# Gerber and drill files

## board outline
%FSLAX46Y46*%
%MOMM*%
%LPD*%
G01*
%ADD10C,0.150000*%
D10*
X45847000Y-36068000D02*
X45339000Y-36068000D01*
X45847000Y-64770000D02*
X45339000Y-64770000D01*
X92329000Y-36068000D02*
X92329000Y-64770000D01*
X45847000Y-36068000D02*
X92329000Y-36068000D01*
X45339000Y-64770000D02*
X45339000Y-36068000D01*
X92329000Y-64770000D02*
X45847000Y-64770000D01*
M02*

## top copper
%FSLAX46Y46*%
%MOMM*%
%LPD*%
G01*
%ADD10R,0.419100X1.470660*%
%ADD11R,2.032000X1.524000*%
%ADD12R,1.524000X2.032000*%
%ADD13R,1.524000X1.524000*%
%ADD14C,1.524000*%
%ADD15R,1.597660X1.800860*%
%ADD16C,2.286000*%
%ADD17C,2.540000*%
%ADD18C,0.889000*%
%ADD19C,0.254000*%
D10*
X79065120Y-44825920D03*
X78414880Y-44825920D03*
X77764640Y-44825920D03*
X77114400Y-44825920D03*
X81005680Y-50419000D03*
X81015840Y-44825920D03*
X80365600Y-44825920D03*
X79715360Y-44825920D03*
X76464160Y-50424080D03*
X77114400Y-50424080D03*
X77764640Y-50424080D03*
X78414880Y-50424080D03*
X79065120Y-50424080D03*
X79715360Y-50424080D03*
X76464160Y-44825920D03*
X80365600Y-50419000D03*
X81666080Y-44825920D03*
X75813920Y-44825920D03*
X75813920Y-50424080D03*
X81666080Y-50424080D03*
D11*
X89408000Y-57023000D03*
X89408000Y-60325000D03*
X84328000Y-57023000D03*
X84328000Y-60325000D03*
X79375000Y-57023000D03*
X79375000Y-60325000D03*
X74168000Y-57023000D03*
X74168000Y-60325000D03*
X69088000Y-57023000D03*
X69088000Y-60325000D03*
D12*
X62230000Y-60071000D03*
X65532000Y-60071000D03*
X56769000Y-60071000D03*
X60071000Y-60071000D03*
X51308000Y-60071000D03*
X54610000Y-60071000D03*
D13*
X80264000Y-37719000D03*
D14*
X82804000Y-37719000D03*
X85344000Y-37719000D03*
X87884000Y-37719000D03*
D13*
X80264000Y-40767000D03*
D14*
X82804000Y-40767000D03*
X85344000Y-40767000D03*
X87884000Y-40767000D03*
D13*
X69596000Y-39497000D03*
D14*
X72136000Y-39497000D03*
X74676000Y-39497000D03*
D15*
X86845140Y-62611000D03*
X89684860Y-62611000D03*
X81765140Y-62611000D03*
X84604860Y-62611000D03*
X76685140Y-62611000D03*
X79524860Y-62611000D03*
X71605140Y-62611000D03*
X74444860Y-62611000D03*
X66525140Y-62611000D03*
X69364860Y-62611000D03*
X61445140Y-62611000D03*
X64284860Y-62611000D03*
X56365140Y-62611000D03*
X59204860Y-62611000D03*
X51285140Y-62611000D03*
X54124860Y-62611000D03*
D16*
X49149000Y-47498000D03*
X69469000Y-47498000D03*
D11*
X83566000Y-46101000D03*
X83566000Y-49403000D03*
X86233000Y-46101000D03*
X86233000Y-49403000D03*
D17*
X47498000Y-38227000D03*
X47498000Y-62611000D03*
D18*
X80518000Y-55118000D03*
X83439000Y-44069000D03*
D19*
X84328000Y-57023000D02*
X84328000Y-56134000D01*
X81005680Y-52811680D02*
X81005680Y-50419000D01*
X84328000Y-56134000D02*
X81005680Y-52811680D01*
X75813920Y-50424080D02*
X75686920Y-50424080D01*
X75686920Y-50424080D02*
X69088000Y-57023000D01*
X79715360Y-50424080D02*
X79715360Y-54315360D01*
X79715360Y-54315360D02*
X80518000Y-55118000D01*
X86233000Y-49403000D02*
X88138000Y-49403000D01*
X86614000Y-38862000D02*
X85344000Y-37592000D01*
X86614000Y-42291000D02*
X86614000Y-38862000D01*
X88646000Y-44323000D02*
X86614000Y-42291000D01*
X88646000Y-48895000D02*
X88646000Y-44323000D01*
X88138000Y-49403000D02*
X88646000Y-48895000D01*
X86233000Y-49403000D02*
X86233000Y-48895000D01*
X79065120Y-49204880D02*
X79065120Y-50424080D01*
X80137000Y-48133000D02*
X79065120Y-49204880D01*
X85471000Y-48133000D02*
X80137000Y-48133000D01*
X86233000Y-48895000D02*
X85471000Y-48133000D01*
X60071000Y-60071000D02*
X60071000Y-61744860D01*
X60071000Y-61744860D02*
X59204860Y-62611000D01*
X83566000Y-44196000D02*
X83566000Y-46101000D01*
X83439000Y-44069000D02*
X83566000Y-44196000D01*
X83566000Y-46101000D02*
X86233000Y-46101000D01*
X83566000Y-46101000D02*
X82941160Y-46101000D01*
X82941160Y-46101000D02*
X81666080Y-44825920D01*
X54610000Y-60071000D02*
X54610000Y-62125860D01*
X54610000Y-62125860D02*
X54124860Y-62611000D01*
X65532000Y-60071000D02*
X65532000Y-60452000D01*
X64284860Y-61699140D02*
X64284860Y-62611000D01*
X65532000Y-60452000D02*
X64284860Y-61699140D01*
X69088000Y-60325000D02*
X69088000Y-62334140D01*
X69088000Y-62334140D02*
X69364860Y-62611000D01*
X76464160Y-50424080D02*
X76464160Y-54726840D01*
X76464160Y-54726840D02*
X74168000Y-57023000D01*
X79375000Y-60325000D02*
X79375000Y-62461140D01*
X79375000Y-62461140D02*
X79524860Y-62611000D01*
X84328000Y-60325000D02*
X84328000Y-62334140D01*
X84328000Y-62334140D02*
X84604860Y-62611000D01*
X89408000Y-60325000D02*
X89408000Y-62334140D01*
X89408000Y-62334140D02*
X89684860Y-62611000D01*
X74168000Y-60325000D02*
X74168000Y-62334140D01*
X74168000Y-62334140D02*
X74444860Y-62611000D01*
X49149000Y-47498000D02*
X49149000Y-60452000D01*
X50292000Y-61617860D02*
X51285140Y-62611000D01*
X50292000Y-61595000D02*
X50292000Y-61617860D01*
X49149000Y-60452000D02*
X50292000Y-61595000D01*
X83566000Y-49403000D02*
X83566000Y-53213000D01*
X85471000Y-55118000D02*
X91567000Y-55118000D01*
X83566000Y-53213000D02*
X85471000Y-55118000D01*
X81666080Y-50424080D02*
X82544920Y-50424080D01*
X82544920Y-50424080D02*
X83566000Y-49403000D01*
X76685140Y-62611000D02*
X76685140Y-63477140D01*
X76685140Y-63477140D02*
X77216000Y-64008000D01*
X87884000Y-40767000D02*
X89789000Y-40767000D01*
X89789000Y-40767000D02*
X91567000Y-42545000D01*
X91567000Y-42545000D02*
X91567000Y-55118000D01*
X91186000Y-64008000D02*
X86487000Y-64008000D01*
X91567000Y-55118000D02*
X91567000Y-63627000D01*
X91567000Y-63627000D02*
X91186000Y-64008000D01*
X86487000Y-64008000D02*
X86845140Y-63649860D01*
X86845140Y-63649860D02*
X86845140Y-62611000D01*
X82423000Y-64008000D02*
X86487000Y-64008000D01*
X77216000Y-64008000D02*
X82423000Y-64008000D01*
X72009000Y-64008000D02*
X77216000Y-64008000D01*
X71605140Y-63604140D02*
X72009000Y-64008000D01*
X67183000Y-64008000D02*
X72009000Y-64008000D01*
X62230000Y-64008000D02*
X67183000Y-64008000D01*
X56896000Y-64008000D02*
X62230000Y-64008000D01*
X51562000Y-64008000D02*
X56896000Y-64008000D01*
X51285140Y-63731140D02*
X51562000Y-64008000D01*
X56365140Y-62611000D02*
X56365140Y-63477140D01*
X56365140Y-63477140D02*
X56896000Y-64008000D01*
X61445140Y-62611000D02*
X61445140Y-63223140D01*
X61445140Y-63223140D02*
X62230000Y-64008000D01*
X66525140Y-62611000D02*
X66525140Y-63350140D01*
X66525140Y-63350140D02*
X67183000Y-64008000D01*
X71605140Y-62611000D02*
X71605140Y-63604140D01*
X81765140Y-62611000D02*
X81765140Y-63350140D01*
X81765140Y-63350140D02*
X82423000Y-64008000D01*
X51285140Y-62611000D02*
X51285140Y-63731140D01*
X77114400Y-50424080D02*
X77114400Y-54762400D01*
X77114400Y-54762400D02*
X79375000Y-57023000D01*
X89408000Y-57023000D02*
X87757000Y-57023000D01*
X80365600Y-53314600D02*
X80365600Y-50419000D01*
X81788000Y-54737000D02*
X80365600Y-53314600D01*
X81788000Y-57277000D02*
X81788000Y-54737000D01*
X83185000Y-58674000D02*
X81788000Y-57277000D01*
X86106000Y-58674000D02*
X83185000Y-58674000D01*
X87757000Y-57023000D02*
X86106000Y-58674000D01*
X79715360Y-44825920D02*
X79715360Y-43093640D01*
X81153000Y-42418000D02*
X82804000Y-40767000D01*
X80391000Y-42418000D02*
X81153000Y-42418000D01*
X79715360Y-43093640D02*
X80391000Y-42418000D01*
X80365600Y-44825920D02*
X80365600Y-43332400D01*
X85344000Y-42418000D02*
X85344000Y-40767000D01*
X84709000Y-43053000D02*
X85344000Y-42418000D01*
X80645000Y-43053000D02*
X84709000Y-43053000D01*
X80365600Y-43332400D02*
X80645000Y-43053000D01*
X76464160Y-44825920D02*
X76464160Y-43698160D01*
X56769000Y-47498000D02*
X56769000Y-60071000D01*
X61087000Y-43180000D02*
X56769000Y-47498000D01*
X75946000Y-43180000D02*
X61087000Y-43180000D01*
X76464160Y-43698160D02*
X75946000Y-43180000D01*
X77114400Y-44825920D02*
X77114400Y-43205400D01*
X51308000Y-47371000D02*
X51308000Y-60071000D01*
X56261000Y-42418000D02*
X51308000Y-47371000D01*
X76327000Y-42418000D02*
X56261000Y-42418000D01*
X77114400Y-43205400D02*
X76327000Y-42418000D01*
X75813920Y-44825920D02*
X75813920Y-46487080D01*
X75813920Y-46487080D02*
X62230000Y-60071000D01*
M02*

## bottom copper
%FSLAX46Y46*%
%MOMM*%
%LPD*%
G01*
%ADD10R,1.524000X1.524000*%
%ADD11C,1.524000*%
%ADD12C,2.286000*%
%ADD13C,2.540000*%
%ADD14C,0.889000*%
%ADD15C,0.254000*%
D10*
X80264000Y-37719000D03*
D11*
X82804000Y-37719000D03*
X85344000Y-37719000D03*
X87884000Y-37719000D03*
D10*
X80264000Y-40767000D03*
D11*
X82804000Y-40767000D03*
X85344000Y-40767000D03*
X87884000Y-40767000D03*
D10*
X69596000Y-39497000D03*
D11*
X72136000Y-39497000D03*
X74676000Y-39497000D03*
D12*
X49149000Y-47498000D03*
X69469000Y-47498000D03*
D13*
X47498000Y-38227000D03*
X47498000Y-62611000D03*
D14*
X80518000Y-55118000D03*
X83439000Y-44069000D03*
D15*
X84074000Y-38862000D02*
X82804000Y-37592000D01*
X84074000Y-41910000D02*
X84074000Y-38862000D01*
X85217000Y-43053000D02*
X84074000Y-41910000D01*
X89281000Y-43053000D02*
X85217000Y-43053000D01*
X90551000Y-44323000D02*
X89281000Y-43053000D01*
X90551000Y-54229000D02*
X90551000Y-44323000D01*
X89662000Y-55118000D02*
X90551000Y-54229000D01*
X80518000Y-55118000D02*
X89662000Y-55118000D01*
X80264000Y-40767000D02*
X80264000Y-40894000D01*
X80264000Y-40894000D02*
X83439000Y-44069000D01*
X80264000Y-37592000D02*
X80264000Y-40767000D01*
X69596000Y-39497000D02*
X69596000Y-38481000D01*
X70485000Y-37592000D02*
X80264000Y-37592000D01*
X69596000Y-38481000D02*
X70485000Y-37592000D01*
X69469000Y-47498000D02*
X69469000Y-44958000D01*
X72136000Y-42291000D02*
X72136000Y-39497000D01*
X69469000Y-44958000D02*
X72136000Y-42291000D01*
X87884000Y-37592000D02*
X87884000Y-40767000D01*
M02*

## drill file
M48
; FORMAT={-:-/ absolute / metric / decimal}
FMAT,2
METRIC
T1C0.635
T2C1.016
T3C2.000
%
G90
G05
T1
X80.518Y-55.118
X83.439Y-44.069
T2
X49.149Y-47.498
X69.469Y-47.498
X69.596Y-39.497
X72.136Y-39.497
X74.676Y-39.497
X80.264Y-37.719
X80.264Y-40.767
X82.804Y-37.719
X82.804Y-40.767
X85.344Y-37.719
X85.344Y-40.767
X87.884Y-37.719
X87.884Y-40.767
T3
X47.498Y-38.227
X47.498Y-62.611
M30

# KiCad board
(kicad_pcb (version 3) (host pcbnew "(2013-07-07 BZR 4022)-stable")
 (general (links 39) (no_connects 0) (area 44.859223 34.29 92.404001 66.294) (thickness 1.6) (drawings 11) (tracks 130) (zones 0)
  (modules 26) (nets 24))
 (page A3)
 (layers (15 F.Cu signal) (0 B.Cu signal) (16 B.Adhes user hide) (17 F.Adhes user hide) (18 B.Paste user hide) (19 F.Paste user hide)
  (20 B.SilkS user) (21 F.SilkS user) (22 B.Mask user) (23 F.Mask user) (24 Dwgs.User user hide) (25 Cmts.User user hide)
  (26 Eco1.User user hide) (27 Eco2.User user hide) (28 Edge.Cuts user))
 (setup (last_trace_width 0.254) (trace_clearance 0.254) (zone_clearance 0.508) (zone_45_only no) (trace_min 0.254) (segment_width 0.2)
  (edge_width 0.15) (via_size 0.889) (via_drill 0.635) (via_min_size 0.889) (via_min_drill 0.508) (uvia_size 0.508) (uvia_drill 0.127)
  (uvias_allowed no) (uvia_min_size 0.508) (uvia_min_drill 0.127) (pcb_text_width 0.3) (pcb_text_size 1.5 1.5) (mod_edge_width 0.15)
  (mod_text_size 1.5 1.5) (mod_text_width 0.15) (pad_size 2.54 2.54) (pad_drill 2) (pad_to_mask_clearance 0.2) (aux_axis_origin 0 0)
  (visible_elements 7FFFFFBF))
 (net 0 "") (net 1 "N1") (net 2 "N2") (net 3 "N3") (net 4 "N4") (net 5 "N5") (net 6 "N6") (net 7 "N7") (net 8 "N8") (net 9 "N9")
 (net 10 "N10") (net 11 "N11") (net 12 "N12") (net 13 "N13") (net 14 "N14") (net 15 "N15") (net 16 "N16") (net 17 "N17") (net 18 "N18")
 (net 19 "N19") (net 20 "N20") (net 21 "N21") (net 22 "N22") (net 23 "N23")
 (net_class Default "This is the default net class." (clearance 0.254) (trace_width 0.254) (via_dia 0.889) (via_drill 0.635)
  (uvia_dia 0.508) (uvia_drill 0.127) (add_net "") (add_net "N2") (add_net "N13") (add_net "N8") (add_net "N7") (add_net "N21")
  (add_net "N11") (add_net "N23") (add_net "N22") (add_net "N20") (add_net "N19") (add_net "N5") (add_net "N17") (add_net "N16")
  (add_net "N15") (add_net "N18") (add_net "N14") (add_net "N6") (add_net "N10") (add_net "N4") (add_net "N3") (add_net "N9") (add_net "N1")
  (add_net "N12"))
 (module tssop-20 (layer F.Cu) (at 78.74 47.625 180)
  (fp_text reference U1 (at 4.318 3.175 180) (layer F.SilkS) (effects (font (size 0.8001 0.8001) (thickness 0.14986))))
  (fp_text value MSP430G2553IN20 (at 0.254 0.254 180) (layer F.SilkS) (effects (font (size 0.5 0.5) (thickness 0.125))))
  (pad 5 smd rect (at -0.32512 2.79908 180) (size 0.4191 1.47066) (layers F.Cu F.Paste F.Mask))
  (pad 6 smd rect (at 0.32512 2.79908 180) (size 0.4191 1.47066) (layers F.Cu F.Paste F.Mask))
  (pad 7 smd rect (at 0.97536 2.79908 180) (size 0.4191 1.47066) (layers F.Cu F.Paste F.Mask))
  (pad 8 smd rect (at 1.6256 2.79908 180) (size 0.4191 1.47066) (layers F.Cu F.Paste F.Mask) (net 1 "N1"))
  (pad 19 smd rect (at -2.26568 -2.794 180) (size 0.4191 1.47066) (layers F.Cu F.Paste F.Mask) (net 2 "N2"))
  (pad 2 smd rect (at -2.27584 2.79908 180) (size 0.4191 1.47066) (layers F.Cu F.Paste F.Mask))
  (pad 3 smd rect (at -1.6256 2.79908 180) (size 0.4191 1.47066) (layers F.Cu F.Paste F.Mask) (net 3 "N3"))
  (pad 4 smd rect (at -0.97536 2.79908 180) (size 0.4191 1.47066) (layers F.Cu F.Paste F.Mask) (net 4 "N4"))
  (pad 12 smd rect (at 2.27584 -2.79908 180) (size 0.4191 1.47066) (layers F.Cu F.Paste F.Mask) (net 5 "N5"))
  (pad 13 smd rect (at 1.6256 -2.79908 180) (size 0.4191 1.47066) (layers F.Cu F.Paste F.Mask) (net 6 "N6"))
  (pad 14 smd rect (at 0.97536 -2.79908 180) (size 0.4191 1.47066) (layers F.Cu F.Paste F.Mask))
  (pad 15 smd rect (at 0.32512 -2.79908 180) (size 0.4191 1.47066) (layers F.Cu F.Paste F.Mask))
  (pad 16 smd rect (at -0.32512 -2.79908 180) (size 0.4191 1.47066) (layers F.Cu F.Paste F.Mask) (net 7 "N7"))
  (pad 17 smd rect (at -0.97536 -2.79908 180) (size 0.4191 1.47066) (layers F.Cu F.Paste F.Mask) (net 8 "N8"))
  (pad 9 smd rect (at 2.27584 2.79908 180) (size 0.4191 1.47066) (layers F.Cu F.Paste F.Mask) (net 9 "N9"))
  (pad 18 smd rect (at -1.6256 -2.794 180) (size 0.4191 1.47066) (layers F.Cu F.Paste F.Mask) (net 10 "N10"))
  (pad 1 smd rect (at -2.92608 2.79908 180) (size 0.4191 1.47066) (layers F.Cu F.Paste F.Mask) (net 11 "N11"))
  (pad 10 smd rect (at 2.92608 2.79908 180) (size 0.4191 1.47066) (layers F.Cu F.Paste F.Mask) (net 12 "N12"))
  (pad 11 smd rect (at 2.92608 -2.79908 180) (size 0.4191 1.47066) (layers F.Cu F.Paste F.Mask) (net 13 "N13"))
  (pad 20 smd rect (at -2.92608 -2.79908 180) (size 0.4191 1.47066) (layers F.Cu F.Paste F.Mask) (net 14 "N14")))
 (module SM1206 (layer F.Cu) (at 89.408 58.674 270)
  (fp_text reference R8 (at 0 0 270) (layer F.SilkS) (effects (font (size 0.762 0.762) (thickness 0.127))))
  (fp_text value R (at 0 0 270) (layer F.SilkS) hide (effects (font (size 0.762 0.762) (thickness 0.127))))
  (pad 1 smd rect (at -1.651 0 270) (size 1.524 2.032) (layers F.Cu F.Paste F.Mask) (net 10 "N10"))
  (pad 2 smd rect (at 1.651 0 270) (size 1.524 2.032) (layers F.Cu F.Paste F.Mask) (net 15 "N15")))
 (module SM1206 (layer F.Cu) (at 84.328 58.674 270)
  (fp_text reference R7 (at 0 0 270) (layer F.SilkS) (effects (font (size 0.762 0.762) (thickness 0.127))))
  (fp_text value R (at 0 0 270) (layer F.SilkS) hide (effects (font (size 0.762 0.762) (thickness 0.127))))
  (pad 1 smd rect (at -1.651 0 270) (size 1.524 2.032) (layers F.Cu F.Paste F.Mask) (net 2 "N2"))
  (pad 2 smd rect (at 1.651 0 270) (size 1.524 2.032) (layers F.Cu F.Paste F.Mask) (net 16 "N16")))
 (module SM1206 (layer F.Cu) (at 79.375 58.674 270)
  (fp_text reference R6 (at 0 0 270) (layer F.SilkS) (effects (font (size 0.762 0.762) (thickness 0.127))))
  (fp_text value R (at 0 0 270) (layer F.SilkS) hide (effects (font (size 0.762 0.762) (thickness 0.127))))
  (pad 1 smd rect (at -1.651 0 270) (size 1.524 2.032) (layers F.Cu F.Paste F.Mask) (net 6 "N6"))
  (pad 2 smd rect (at 1.651 0 270) (size 1.524 2.032) (layers F.Cu F.Paste F.Mask) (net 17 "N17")))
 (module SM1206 (layer F.Cu) (at 74.168 58.674 270)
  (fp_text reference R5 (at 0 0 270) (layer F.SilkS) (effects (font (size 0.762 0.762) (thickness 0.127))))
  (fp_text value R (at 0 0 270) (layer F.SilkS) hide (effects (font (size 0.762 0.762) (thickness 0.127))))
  (pad 1 smd rect (at -1.651 0 270) (size 1.524 2.032) (layers F.Cu F.Paste F.Mask) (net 5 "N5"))
  (pad 2 smd rect (at 1.651 0 270) (size 1.524 2.032) (layers F.Cu F.Paste F.Mask) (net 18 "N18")))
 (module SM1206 (layer F.Cu) (at 69.088 58.674 270)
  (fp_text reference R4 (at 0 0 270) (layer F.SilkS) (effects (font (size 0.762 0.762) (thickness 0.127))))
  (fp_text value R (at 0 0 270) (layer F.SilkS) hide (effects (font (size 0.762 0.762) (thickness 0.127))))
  (pad 1 smd rect (at -1.651 0 270) (size 1.524 2.032) (layers F.Cu F.Paste F.Mask) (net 13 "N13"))
  (pad 2 smd rect (at 1.651 0 270) (size 1.524 2.032) (layers F.Cu F.Paste F.Mask) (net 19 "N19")))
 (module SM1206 (layer F.Cu) (at 63.881 60.071)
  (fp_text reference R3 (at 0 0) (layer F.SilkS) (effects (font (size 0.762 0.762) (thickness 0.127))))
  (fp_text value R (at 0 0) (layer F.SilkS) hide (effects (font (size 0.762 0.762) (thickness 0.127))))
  (pad 1 smd rect (at -1.651 0) (size 1.524 2.032) (layers F.Cu F.Paste F.Mask) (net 12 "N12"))
  (pad 2 smd rect (at 1.651 0) (size 1.524 2.032) (layers F.Cu F.Paste F.Mask) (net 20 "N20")))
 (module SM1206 (layer F.Cu) (at 58.42 60.071)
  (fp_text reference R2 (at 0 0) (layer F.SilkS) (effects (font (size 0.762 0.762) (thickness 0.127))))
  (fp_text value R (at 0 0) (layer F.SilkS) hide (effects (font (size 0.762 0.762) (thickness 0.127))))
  (pad 1 smd rect (at -1.651 0) (size 1.524 2.032) (layers F.Cu F.Paste F.Mask) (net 9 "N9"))
  (pad 2 smd rect (at 1.651 0) (size 1.524 2.032) (layers F.Cu F.Paste F.Mask) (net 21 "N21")))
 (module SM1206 (layer F.Cu) (at 52.959 60.071)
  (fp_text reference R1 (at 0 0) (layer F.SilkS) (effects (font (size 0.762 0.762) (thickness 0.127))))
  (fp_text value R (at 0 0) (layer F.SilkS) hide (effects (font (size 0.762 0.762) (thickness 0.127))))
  (pad 1 smd rect (at -1.651 0) (size 1.524 2.032) (layers F.Cu F.Paste F.Mask) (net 1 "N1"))
  (pad 2 smd rect (at 1.651 0) (size 1.524 2.032) (layers F.Cu F.Paste F.Mask) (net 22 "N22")))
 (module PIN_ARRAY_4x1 (layer F.Cu) (at 84.074 37.719)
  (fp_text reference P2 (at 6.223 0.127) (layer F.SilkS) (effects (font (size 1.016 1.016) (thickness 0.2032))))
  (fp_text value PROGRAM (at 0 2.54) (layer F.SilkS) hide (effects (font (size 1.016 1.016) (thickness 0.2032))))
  (pad 1 thru_hole rect (at -3.81 0) (size 1.524 1.524) (drill 1.016) (layers *.Cu *.Mask F.SilkS) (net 11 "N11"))
  (pad 2 thru_hole circle (at -1.27 0) (size 1.524 1.524) (drill 1.016) (layers *.Cu *.Mask F.SilkS) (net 8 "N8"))
  (pad 3 thru_hole circle (at 1.27 0) (size 1.524 1.524) (drill 1.016) (layers *.Cu *.Mask F.SilkS) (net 7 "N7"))
  (pad 4 thru_hole circle (at 3.81 0) (size 1.524 1.524) (drill 1.016) (layers *.Cu *.Mask F.SilkS) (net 14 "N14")))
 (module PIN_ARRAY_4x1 (layer F.Cu) (at 84.074 40.767)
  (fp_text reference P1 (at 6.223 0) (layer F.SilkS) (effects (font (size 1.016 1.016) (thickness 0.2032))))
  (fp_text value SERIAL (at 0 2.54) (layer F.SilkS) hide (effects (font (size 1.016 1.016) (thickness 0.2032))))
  (pad 1 thru_hole rect (at -3.81 0) (size 1.524 1.524) (drill 1.016) (layers *.Cu *.Mask F.SilkS) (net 11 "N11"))
  (pad 2 thru_hole circle (at -1.27 0) (size 1.524 1.524) (drill 1.016) (layers *.Cu *.Mask F.SilkS) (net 4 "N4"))
  (pad 3 thru_hole circle (at 1.27 0) (size 1.524 1.524) (drill 1.016) (layers *.Cu *.Mask F.SilkS) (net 3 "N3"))
  (pad 4 thru_hole circle (at 3.81 0) (size 1.524 1.524) (drill 1.016) (layers *.Cu *.Mask F.SilkS) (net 14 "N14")))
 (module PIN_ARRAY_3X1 (layer F.Cu) (at 72.136 39.497)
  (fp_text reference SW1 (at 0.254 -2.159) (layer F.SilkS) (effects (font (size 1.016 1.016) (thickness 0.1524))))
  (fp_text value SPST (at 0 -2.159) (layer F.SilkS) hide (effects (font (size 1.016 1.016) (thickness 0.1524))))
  (pad 1 thru_hole rect (at -2.54 0) (size 1.524 1.524) (drill 1.016) (layers *.Cu *.Mask F.SilkS) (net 11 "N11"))
  (pad 2 thru_hole circle (at 0 0) (size 1.524 1.524) (drill 1.016) (layers *.Cu *.Mask F.SilkS) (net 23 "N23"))
  (pad 3 thru_hole circle (at 2.54 0) (size 1.524 1.524) (drill 1.016) (layers *.Cu *.Mask F.SilkS)))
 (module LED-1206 (layer F.Cu) (at 88.265 62.611)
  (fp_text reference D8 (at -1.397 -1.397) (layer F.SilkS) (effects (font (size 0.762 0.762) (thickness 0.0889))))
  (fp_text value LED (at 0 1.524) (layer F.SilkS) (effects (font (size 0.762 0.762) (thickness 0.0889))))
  (pad 1 smd rect (at -1.41986 0) (size 1.59766 1.80086) (layers F.Cu F.Paste F.Mask) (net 14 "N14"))
  (pad 2 smd rect (at 1.41986 0) (size 1.59766 1.80086) (layers F.Cu F.Paste F.Mask) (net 15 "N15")))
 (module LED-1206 (layer F.Cu) (at 83.185 62.611)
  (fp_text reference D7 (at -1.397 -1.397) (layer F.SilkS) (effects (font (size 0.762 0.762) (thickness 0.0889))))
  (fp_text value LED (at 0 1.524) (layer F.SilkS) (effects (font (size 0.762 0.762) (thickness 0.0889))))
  (pad 1 smd rect (at -1.41986 0) (size 1.59766 1.80086) (layers F.Cu F.Paste F.Mask) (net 14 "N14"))
  (pad 2 smd rect (at 1.41986 0) (size 1.59766 1.80086) (layers F.Cu F.Paste F.Mask) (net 16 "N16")))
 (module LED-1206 (layer F.Cu) (at 78.105 62.611)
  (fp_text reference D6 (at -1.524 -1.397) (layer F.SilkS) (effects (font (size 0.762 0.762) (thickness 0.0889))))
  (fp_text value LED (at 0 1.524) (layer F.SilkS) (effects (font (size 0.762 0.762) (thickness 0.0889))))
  (pad 1 smd rect (at -1.41986 0) (size 1.59766 1.80086) (layers F.Cu F.Paste F.Mask) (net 14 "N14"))
  (pad 2 smd rect (at 1.41986 0) (size 1.59766 1.80086) (layers F.Cu F.Paste F.Mask) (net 17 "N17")))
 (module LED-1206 (layer F.Cu) (at 73.025 62.611)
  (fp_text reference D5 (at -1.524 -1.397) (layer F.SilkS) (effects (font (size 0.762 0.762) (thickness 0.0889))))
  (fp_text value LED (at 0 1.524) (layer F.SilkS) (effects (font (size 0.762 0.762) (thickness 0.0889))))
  (pad 1 smd rect (at -1.41986 0) (size 1.59766 1.80086) (layers F.Cu F.Paste F.Mask) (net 14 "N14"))
  (pad 2 smd rect (at 1.41986 0) (size 1.59766 1.80086) (layers F.Cu F.Paste F.Mask) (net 18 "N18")))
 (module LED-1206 (layer F.Cu) (at 67.945 62.611)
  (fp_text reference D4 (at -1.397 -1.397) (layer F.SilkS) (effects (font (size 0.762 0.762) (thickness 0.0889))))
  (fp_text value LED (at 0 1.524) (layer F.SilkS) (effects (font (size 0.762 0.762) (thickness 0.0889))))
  (pad 1 smd rect (at -1.41986 0) (size 1.59766 1.80086) (layers F.Cu F.Paste F.Mask) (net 14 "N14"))
  (pad 2 smd rect (at 1.41986 0) (size 1.59766 1.80086) (layers F.Cu F.Paste F.Mask) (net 19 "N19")))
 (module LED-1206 (layer F.Cu) (at 62.865 62.611)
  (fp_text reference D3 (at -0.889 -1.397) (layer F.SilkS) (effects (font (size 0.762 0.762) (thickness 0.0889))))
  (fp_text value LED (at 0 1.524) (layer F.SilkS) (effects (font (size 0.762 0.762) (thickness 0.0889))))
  (pad 1 smd rect (at -1.41986 0) (size 1.59766 1.80086) (layers F.Cu F.Paste F.Mask) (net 14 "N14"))
  (pad 2 smd rect (at 1.41986 0) (size 1.59766 1.80086) (layers F.Cu F.Paste F.Mask) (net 20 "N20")))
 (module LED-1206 (layer F.Cu) (at 57.785 62.611)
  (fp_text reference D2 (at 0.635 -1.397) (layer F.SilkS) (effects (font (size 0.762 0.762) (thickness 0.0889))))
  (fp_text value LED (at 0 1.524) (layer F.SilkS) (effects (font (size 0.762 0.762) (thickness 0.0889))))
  (pad 1 smd rect (at -1.41986 0) (size 1.59766 1.80086) (layers F.Cu F.Paste F.Mask) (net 14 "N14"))
  (pad 2 smd rect (at 1.41986 0) (size 1.59766 1.80086) (layers F.Cu F.Paste F.Mask) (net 21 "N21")))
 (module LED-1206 (layer F.Cu) (at 52.705 62.611)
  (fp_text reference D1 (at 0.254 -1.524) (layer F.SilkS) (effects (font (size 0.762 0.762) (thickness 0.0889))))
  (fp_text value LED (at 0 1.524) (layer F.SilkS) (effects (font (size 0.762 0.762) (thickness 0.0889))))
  (pad 1 smd rect (at -1.41986 0) (size 1.59766 1.80086) (layers F.Cu F.Paste F.Mask) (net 14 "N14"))
  (pad 2 smd rect (at 1.41986 0) (size 1.59766 1.80086) (layers F.Cu F.Paste F.Mask) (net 22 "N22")))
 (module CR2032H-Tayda (layer F.Cu) (at 56.769 47.498)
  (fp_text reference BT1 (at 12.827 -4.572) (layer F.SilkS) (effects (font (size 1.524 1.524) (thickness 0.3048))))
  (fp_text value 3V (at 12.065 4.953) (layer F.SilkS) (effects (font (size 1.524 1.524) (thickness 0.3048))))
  (pad 2 thru_hole circle (at -7.62 0) (size 2.286 2.286) (drill 1.016) (layers *.Cu *.Mask F.SilkS) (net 14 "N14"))
  (pad 1 thru_hole circle (at 12.7 0) (size 2.286 2.286) (drill 1.016) (layers *.Cu *.Mask F.SilkS) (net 23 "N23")))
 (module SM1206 (layer F.Cu) (at 83.566 47.752 270)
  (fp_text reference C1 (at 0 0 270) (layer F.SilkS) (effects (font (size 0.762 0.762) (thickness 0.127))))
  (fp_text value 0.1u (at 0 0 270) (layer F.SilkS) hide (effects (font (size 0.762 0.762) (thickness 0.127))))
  (pad 1 smd rect (at -1.651 0 270) (size 1.524 2.032) (layers F.Cu F.Paste F.Mask) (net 11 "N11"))
  (pad 2 smd rect (at 1.651 0 270) (size 1.524 2.032) (layers F.Cu F.Paste F.Mask) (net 14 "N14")))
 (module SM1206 (layer F.Cu) (at 86.233 47.752 270)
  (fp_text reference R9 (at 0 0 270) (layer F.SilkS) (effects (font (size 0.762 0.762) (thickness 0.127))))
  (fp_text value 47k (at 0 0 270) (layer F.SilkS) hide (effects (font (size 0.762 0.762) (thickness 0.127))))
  (pad 1 smd rect (at -1.651 0 270) (size 1.524 2.032) (layers F.Cu F.Paste F.Mask) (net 11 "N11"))
  (pad 2 smd rect (at 1.651 0 270) (size 1.524 2.032) (layers F.Cu F.Paste F.Mask) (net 7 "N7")))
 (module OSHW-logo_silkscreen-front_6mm (layer F.Cu) (at 56.261 51.816)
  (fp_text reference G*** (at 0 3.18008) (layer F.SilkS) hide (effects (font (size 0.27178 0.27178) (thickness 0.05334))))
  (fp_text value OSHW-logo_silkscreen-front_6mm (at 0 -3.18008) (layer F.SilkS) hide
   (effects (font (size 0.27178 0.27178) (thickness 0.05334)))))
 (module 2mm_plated (layer F.Cu) (at 47.498 38.227)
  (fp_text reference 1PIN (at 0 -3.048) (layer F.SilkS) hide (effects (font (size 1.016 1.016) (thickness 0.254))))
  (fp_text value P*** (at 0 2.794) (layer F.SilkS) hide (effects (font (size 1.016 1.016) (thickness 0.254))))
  (pad "" thru_hole circle (at 0 0) (size 2.54 2.54) (drill 2) (layers *.Cu *.Mask F.SilkS)))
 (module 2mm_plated (layer F.Cu) (at 47.498 62.611)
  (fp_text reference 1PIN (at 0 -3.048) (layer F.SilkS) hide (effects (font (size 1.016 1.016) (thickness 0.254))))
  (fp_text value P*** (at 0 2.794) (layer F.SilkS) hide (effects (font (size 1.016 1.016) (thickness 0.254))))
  (pad "" thru_hole circle (at 0 0) (size 2.54 2.54) (drill 2) (layers *.Cu *.Mask F.SilkS)))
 (gr_line (start 45.847 36.068) (end 45.339 36.068) (angle 90) (layer Edge.Cuts) (width 0.15))
 (gr_line (start 45.847 64.77) (end 45.339 64.77) (angle 90) (layer Edge.Cuts) (width 0.15))
 (gr_line (start 92.329 36.068) (end 92.329 64.77) (angle 90) (layer Edge.Cuts) (width 0.15))
 (gr_line (start 45.847 36.068) (end 92.329 36.068) (angle 90) (layer Edge.Cuts) (width 0.15))
 (gr_line (start 45.339 64.77) (end 45.339 36.068) (angle 90) (layer Edge.Cuts) (width 0.15))
 (gr_line (start 92.329 64.77) (end 45.847 64.77) (angle 90) (layer Edge.Cuts) (width 0.15))
 (segment (start 84.328 57.023) (end 84.328 56.134) (width 0.254) (layer F.Cu) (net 2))
 (segment (start 81.00568 52.81168) (end 81.00568 50.419) (width 0.254) (layer F.Cu) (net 2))
 (segment (start 84.328 56.134) (end 81.00568 52.81168) (width 0.254) (layer F.Cu) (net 2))
 (segment (start 75.81392 50.42408) (end 75.68692 50.42408) (width 0.254) (layer F.Cu) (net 13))
 (segment (start 75.68692 50.42408) (end 69.088 57.023) (width 0.254) (layer F.Cu) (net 13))
 (segment (start 79.71536 50.42408) (end 79.71536 54.31536) (width 0.254) (layer F.Cu) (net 8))
 (segment (start 84.074 38.862) (end 82.804 37.592) (width 0.254) (layer B.Cu) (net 8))
 (segment (start 84.074 41.91) (end 84.074 38.862) (width 0.254) (layer B.Cu) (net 8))
 (segment (start 85.217 43.053) (end 84.074 41.91) (width 0.254) (layer B.Cu) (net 8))
 (segment (start 89.281 43.053) (end 85.217 43.053) (width 0.254) (layer B.Cu) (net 8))
 (segment (start 90.551 44.323) (end 89.281 43.053) (width 0.254) (layer B.Cu) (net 8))
 (segment (start 90.551 54.229) (end 90.551 44.323) (width 0.254) (layer B.Cu) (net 8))
 (segment (start 89.662 55.118) (end 90.551 54.229) (width 0.254) (layer B.Cu) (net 8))
 (segment (start 80.518 55.118) (end 89.662 55.118) (width 0.254) (layer B.Cu) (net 8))
 (via (at 80.518 55.118) (size 0.889) (layers F.Cu B.Cu) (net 8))
 (segment (start 79.71536 54.31536) (end 80.518 55.118) (width 0.254) (layer F.Cu) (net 8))
 (segment (start 86.233 49.403) (end 88.138 49.403) (width 0.254) (layer F.Cu) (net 7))
 (segment (start 86.614 38.862) (end 85.344 37.592) (width 0.254) (layer F.Cu) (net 7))
 (segment (start 86.614 42.291) (end 86.614 38.862) (width 0.254) (layer F.Cu) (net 7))
 (segment (start 88.646 44.323) (end 86.614 42.291) (width 0.254) (layer F.Cu) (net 7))
 (segment (start 88.646 48.895) (end 88.646 44.323) (width 0.254) (layer F.Cu) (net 7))
 (segment (start 88.138 49.403) (end 88.646 48.895) (width 0.254) (layer F.Cu) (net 7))
 (segment (start 86.233 49.403) (end 86.233 48.895) (width 0.254) (layer F.Cu) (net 7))
 (segment (start 79.06512 49.20488) (end 79.06512 50.42408) (width 0.254) (layer F.Cu) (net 7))
 (segment (start 80.137 48.133) (end 79.06512 49.20488) (width 0.254) (layer F.Cu) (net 7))
 (segment (start 85.471 48.133) (end 80.137 48.133) (width 0.254) (layer F.Cu) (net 7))
 (segment (start 86.233 48.895) (end 85.471 48.133) (width 0.254) (layer F.Cu) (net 7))
 (segment (start 60.071 60.071) (end 60.071 61.74486) (width 0.254) (layer F.Cu) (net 21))
 (segment (start 60.071 61.74486) (end 59.20486 62.611) (width 0.254) (layer F.Cu) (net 21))
 (segment (start 80.264 40.767) (end 80.264 40.894) (width 0.254) (layer B.Cu) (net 11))
 (segment (start 83.566 44.196) (end 83.566 46.101) (width 0.254) (layer F.Cu) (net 11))
 (segment (start 83.439 44.069) (end 83.566 44.196) (width 0.254) (layer F.Cu) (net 11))
 (via (at 83.439 44.069) (size 0.889) (layers F.Cu B.Cu) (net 11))
 (segment (start 80.264 40.894) (end 83.439 44.069) (width 0.254) (layer B.Cu) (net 11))
 (segment (start 83.566 46.101) (end 86.233 46.101) (width 0.254) (layer F.Cu) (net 11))
 (segment (start 83.566 46.101) (end 82.94116 46.101) (width 0.254) (layer F.Cu) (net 11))
 (segment (start 82.94116 46.101) (end 81.66608 44.82592) (width 0.254) (layer F.Cu) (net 11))
 (segment (start 80.264 37.592) (end 80.264 40.767) (width 0.254) (layer B.Cu) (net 11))
 (segment (start 69.596 39.497) (end 69.596 38.481) (width 0.254) (layer B.Cu) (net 11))
 (segment (start 70.485 37.592) (end 80.264 37.592) (width 0.254) (layer B.Cu) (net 11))
 (segment (start 69.596 38.481) (end 70.485 37.592) (width 0.254) (layer B.Cu) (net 11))
 (segment (start 69.469 47.498) (end 69.469 44.958) (width 0.254) (layer B.Cu) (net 23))
 (segment (start 72.136 42.291) (end 72.136 39.497) (width 0.254) (layer B.Cu) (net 23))
 (segment (start 69.469 44.958) (end 72.136 42.291) (width 0.254) (layer B.Cu) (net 23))
 (segment (start 54.61 60.071) (end 54.61 62.12586) (width 0.254) (layer F.Cu) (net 22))
 (segment (start 54.61 62.12586) (end 54.12486 62.611) (width 0.254) (layer F.Cu) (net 22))
 (segment (start 65.532 60.071) (end 65.532 60.452) (width 0.254) (layer F.Cu) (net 20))
 (segment (start 64.28486 61.69914) (end 64.28486 62.611) (width 0.254) (layer F.Cu) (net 20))
 (segment (start 65.532 60.452) (end 64.28486 61.69914) (width 0.254) (layer F.Cu) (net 20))
 (segment (start 69.088 60.325) (end 69.088 62.33414) (width 0.254) (layer F.Cu) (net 19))
 (segment (start 69.088 62.33414) (end 69.36486 62.611) (width 0.254) (layer F.Cu) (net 19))
 (segment (start 76.46416 50.42408) (end 76.46416 54.72684) (width 0.254) (layer F.Cu) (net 5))
 (segment (start 76.46416 54.72684) (end 74.168 57.023) (width 0.254) (layer F.Cu) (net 5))
 (segment (start 79.375 60.325) (end 79.375 62.46114) (width 0.254) (layer F.Cu) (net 17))
 (segment (start 79.375 62.46114) (end 79.52486 62.611) (width 0.254) (layer F.Cu) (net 17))
 (segment (start 84.328 60.325) (end 84.328 62.33414) (width 0.254) (layer F.Cu) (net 16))
 (segment (start 84.328 62.33414) (end 84.60486 62.611) (width 0.254) (layer F.Cu) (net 16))
 (segment (start 89.408 60.325) (end 89.408 62.33414) (width 0.254) (layer F.Cu) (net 15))
 (segment (start 89.408 62.33414) (end 89.68486 62.611) (width 0.254) (layer F.Cu) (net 15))
 (segment (start 74.168 60.325) (end 74.168 62.33414) (width 0.254) (layer F.Cu) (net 18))
 (segment (start 74.168 62.33414) (end 74.44486 62.611) (width 0.254) (layer F.Cu) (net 18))
 (segment (start 49.149 47.498) (end 49.149 60.452) (width 0.254) (layer F.Cu) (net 14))
 (segment (start 50.292 61.61786) (end 51.28514 62.611) (width 0.254) (layer F.Cu) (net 14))
 (segment (start 50.292 61.595) (end 50.292 61.61786) (width 0.254) (layer F.Cu) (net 14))
 (segment (start 49.149 60.452) (end 50.292 61.595) (width 0.254) (layer F.Cu) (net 14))
 (segment (start 83.566 49.403) (end 83.566 53.213) (width 0.254) (layer F.Cu) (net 14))
 (segment (start 85.471 55.118) (end 91.567 55.118) (width 0.254) (layer F.Cu) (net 14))
 (segment (start 83.566 53.213) (end 85.471 55.118) (width 0.254) (layer F.Cu) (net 14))
 (segment (start 81.66608 50.42408) (end 82.54492 50.42408) (width 0.254) (layer F.Cu) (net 14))
 (segment (start 82.54492 50.42408) (end 83.566 49.403) (width 0.254) (layer F.Cu) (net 14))
 (segment (start 76.68514 62.611) (end 76.68514 63.47714) (width 0.254) (layer F.Cu) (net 14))
 (segment (start 76.68514 63.47714) (end 77.216 64.008) (width 0.254) (layer F.Cu) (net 14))
 (segment (start 87.884 40.767) (end 89.789 40.767) (width 0.254) (layer F.Cu) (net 14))
 (segment (start 89.789 40.767) (end 91.567 42.545) (width 0.254) (layer F.Cu) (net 14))
 (segment (start 91.567 42.545) (end 91.567 55.118) (width 0.254) (layer F.Cu) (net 14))
 (segment (start 91.186 64.008) (end 86.487 64.008) (width 0.254) (layer F.Cu) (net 14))
 (segment (start 91.567 55.118) (end 91.567 63.627) (width 0.254) (layer F.Cu) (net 14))
 (segment (start 91.567 63.627) (end 91.186 64.008) (width 0.254) (layer F.Cu) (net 14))
 (segment (start 87.884 37.592) (end 87.884 40.767) (width 0.254) (layer B.Cu) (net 14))
 (segment (start 86.487 64.008) (end 86.84514 63.64986) (width 0.254) (layer F.Cu) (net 14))
 (segment (start 86.84514 63.64986) (end 86.84514 62.611) (width 0.254) (layer F.Cu) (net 14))
 (segment (start 82.423 64.008) (end 86.487 64.008) (width 0.254) (layer F.Cu) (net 14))
 (segment (start 77.216 64.008) (end 82.423 64.008) (width 0.254) (layer F.Cu) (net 14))
 (segment (start 72.009 64.008) (end 77.216 64.008) (width 0.254) (layer F.Cu) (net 14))
 (segment (start 71.60514 63.60414) (end 72.009 64.008) (width 0.254) (layer F.Cu) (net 14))
 (segment (start 67.183 64.008) (end 72.009 64.008) (width 0.254) (layer F.Cu) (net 14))
 (segment (start 62.23 64.008) (end 67.183 64.008) (width 0.254) (layer F.Cu) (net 14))
 (segment (start 56.896 64.008) (end 62.23 64.008) (width 0.254) (layer F.Cu) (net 14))
 (segment (start 51.562 64.008) (end 56.896 64.008) (width 0.254) (layer F.Cu) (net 14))
 (segment (start 51.28514 63.73114) (end 51.562 64.008) (width 0.254) (layer F.Cu) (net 14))
 (segment (start 56.36514 62.611) (end 56.36514 63.47714) (width 0.254) (layer F.Cu) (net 14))
 (segment (start 56.36514 63.47714) (end 56.896 64.008) (width 0.254) (layer F.Cu) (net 14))
 (segment (start 61.44514 62.611) (end 61.44514 63.22314) (width 0.254) (layer F.Cu) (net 14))
 (segment (start 61.44514 63.22314) (end 62.23 64.008) (width 0.254) (layer F.Cu) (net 14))
 (segment (start 66.52514 62.611) (end 66.52514 63.35014) (width 0.254) (layer F.Cu) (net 14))
 (segment (start 66.52514 63.35014) (end 67.183 64.008) (width 0.254) (layer F.Cu) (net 14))
 (segment (start 71.60514 62.611) (end 71.60514 63.60414) (width 0.254) (layer F.Cu) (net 14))
 (segment (start 81.76514 62.611) (end 81.76514 63.35014) (width 0.254) (layer F.Cu) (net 14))
 (segment (start 81.76514 63.35014) (end 82.423 64.008) (width 0.254) (layer F.Cu) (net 14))
 (segment (start 51.28514 62.611) (end 51.28514 63.73114) (width 0.254) (layer F.Cu) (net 14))
 (segment (start 77.1144 50.42408) (end 77.1144 54.7624) (width 0.254) (layer F.Cu) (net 6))
 (segment (start 77.1144 54.7624) (end 79.375 57.023) (width 0.254) (layer F.Cu) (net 6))
 (segment (start 89.408 57.023) (end 87.757 57.023) (width 0.254) (layer F.Cu) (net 10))
 (segment (start 80.3656 53.3146) (end 80.3656 50.419) (width 0.254) (layer F.Cu) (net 10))
 (segment (start 81.788 54.737) (end 80.3656 53.3146) (width 0.254) (layer F.Cu) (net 10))
 (segment (start 81.788 57.277) (end 81.788 54.737) (width 0.254) (layer F.Cu) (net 10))
 (segment (start 83.185 58.674) (end 81.788 57.277) (width 0.254) (layer F.Cu) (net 10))
 (segment (start 86.106 58.674) (end 83.185 58.674) (width 0.254) (layer F.Cu) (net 10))
 (segment (start 87.757 57.023) (end 86.106 58.674) (width 0.254) (layer F.Cu) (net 10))
 (segment (start 79.71536 44.82592) (end 79.71536 43.09364) (width 0.254) (layer F.Cu) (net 4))
 (segment (start 81.153 42.418) (end 82.804 40.767) (width 0.254) (layer F.Cu) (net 4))
 (segment (start 80.391 42.418) (end 81.153 42.418) (width 0.254) (layer F.Cu) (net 4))
 (segment (start 79.71536 43.09364) (end 80.391 42.418) (width 0.254) (layer F.Cu) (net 4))
 (segment (start 80.3656 44.82592) (end 80.3656 43.3324) (width 0.254) (layer F.Cu) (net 3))
 (segment (start 85.344 42.418) (end 85.344 40.767) (width 0.254) (layer F.Cu) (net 3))
 (segment (start 84.709 43.053) (end 85.344 42.418) (width 0.254) (layer F.Cu) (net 3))
 (segment (start 80.645 43.053) (end 84.709 43.053) (width 0.254) (layer F.Cu) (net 3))
 (segment (start 80.3656 43.3324) (end 80.645 43.053) (width 0.254) (layer F.Cu) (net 3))
 (segment (start 76.46416 44.82592) (end 76.46416 43.69816) (width 0.254) (layer F.Cu) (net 9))
 (segment (start 56.769 47.498) (end 56.769 60.071) (width 0.254) (layer F.Cu) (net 9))
 (segment (start 61.087 43.18) (end 56.769 47.498) (width 0.254) (layer F.Cu) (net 9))
 (segment (start 75.946 43.18) (end 61.087 43.18) (width 0.254) (layer F.Cu) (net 9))
 (segment (start 76.46416 43.69816) (end 75.946 43.18) (width 0.254) (layer F.Cu) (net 9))
 (segment (start 77.1144 44.82592) (end 77.1144 43.2054) (width 0.254) (layer F.Cu) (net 1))
 (segment (start 51.308 47.371) (end 51.308 60.071) (width 0.254) (layer F.Cu) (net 1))
 (segment (start 56.261 42.418) (end 51.308 47.371) (width 0.254) (layer F.Cu) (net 1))
 (segment (start 76.327 42.418) (end 56.261 42.418) (width 0.254) (layer F.Cu) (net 1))
 (segment (start 77.1144 43.2054) (end 76.327 42.418) (width 0.254) (layer F.Cu) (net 1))
 (segment (start 75.81392 44.82592) (end 75.81392 46.48708) (width 0.254) (layer F.Cu) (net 12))
 (segment (start 75.81392 46.48708) (end 62.23 60.071) (width 0.254) (layer F.Cu) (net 12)))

